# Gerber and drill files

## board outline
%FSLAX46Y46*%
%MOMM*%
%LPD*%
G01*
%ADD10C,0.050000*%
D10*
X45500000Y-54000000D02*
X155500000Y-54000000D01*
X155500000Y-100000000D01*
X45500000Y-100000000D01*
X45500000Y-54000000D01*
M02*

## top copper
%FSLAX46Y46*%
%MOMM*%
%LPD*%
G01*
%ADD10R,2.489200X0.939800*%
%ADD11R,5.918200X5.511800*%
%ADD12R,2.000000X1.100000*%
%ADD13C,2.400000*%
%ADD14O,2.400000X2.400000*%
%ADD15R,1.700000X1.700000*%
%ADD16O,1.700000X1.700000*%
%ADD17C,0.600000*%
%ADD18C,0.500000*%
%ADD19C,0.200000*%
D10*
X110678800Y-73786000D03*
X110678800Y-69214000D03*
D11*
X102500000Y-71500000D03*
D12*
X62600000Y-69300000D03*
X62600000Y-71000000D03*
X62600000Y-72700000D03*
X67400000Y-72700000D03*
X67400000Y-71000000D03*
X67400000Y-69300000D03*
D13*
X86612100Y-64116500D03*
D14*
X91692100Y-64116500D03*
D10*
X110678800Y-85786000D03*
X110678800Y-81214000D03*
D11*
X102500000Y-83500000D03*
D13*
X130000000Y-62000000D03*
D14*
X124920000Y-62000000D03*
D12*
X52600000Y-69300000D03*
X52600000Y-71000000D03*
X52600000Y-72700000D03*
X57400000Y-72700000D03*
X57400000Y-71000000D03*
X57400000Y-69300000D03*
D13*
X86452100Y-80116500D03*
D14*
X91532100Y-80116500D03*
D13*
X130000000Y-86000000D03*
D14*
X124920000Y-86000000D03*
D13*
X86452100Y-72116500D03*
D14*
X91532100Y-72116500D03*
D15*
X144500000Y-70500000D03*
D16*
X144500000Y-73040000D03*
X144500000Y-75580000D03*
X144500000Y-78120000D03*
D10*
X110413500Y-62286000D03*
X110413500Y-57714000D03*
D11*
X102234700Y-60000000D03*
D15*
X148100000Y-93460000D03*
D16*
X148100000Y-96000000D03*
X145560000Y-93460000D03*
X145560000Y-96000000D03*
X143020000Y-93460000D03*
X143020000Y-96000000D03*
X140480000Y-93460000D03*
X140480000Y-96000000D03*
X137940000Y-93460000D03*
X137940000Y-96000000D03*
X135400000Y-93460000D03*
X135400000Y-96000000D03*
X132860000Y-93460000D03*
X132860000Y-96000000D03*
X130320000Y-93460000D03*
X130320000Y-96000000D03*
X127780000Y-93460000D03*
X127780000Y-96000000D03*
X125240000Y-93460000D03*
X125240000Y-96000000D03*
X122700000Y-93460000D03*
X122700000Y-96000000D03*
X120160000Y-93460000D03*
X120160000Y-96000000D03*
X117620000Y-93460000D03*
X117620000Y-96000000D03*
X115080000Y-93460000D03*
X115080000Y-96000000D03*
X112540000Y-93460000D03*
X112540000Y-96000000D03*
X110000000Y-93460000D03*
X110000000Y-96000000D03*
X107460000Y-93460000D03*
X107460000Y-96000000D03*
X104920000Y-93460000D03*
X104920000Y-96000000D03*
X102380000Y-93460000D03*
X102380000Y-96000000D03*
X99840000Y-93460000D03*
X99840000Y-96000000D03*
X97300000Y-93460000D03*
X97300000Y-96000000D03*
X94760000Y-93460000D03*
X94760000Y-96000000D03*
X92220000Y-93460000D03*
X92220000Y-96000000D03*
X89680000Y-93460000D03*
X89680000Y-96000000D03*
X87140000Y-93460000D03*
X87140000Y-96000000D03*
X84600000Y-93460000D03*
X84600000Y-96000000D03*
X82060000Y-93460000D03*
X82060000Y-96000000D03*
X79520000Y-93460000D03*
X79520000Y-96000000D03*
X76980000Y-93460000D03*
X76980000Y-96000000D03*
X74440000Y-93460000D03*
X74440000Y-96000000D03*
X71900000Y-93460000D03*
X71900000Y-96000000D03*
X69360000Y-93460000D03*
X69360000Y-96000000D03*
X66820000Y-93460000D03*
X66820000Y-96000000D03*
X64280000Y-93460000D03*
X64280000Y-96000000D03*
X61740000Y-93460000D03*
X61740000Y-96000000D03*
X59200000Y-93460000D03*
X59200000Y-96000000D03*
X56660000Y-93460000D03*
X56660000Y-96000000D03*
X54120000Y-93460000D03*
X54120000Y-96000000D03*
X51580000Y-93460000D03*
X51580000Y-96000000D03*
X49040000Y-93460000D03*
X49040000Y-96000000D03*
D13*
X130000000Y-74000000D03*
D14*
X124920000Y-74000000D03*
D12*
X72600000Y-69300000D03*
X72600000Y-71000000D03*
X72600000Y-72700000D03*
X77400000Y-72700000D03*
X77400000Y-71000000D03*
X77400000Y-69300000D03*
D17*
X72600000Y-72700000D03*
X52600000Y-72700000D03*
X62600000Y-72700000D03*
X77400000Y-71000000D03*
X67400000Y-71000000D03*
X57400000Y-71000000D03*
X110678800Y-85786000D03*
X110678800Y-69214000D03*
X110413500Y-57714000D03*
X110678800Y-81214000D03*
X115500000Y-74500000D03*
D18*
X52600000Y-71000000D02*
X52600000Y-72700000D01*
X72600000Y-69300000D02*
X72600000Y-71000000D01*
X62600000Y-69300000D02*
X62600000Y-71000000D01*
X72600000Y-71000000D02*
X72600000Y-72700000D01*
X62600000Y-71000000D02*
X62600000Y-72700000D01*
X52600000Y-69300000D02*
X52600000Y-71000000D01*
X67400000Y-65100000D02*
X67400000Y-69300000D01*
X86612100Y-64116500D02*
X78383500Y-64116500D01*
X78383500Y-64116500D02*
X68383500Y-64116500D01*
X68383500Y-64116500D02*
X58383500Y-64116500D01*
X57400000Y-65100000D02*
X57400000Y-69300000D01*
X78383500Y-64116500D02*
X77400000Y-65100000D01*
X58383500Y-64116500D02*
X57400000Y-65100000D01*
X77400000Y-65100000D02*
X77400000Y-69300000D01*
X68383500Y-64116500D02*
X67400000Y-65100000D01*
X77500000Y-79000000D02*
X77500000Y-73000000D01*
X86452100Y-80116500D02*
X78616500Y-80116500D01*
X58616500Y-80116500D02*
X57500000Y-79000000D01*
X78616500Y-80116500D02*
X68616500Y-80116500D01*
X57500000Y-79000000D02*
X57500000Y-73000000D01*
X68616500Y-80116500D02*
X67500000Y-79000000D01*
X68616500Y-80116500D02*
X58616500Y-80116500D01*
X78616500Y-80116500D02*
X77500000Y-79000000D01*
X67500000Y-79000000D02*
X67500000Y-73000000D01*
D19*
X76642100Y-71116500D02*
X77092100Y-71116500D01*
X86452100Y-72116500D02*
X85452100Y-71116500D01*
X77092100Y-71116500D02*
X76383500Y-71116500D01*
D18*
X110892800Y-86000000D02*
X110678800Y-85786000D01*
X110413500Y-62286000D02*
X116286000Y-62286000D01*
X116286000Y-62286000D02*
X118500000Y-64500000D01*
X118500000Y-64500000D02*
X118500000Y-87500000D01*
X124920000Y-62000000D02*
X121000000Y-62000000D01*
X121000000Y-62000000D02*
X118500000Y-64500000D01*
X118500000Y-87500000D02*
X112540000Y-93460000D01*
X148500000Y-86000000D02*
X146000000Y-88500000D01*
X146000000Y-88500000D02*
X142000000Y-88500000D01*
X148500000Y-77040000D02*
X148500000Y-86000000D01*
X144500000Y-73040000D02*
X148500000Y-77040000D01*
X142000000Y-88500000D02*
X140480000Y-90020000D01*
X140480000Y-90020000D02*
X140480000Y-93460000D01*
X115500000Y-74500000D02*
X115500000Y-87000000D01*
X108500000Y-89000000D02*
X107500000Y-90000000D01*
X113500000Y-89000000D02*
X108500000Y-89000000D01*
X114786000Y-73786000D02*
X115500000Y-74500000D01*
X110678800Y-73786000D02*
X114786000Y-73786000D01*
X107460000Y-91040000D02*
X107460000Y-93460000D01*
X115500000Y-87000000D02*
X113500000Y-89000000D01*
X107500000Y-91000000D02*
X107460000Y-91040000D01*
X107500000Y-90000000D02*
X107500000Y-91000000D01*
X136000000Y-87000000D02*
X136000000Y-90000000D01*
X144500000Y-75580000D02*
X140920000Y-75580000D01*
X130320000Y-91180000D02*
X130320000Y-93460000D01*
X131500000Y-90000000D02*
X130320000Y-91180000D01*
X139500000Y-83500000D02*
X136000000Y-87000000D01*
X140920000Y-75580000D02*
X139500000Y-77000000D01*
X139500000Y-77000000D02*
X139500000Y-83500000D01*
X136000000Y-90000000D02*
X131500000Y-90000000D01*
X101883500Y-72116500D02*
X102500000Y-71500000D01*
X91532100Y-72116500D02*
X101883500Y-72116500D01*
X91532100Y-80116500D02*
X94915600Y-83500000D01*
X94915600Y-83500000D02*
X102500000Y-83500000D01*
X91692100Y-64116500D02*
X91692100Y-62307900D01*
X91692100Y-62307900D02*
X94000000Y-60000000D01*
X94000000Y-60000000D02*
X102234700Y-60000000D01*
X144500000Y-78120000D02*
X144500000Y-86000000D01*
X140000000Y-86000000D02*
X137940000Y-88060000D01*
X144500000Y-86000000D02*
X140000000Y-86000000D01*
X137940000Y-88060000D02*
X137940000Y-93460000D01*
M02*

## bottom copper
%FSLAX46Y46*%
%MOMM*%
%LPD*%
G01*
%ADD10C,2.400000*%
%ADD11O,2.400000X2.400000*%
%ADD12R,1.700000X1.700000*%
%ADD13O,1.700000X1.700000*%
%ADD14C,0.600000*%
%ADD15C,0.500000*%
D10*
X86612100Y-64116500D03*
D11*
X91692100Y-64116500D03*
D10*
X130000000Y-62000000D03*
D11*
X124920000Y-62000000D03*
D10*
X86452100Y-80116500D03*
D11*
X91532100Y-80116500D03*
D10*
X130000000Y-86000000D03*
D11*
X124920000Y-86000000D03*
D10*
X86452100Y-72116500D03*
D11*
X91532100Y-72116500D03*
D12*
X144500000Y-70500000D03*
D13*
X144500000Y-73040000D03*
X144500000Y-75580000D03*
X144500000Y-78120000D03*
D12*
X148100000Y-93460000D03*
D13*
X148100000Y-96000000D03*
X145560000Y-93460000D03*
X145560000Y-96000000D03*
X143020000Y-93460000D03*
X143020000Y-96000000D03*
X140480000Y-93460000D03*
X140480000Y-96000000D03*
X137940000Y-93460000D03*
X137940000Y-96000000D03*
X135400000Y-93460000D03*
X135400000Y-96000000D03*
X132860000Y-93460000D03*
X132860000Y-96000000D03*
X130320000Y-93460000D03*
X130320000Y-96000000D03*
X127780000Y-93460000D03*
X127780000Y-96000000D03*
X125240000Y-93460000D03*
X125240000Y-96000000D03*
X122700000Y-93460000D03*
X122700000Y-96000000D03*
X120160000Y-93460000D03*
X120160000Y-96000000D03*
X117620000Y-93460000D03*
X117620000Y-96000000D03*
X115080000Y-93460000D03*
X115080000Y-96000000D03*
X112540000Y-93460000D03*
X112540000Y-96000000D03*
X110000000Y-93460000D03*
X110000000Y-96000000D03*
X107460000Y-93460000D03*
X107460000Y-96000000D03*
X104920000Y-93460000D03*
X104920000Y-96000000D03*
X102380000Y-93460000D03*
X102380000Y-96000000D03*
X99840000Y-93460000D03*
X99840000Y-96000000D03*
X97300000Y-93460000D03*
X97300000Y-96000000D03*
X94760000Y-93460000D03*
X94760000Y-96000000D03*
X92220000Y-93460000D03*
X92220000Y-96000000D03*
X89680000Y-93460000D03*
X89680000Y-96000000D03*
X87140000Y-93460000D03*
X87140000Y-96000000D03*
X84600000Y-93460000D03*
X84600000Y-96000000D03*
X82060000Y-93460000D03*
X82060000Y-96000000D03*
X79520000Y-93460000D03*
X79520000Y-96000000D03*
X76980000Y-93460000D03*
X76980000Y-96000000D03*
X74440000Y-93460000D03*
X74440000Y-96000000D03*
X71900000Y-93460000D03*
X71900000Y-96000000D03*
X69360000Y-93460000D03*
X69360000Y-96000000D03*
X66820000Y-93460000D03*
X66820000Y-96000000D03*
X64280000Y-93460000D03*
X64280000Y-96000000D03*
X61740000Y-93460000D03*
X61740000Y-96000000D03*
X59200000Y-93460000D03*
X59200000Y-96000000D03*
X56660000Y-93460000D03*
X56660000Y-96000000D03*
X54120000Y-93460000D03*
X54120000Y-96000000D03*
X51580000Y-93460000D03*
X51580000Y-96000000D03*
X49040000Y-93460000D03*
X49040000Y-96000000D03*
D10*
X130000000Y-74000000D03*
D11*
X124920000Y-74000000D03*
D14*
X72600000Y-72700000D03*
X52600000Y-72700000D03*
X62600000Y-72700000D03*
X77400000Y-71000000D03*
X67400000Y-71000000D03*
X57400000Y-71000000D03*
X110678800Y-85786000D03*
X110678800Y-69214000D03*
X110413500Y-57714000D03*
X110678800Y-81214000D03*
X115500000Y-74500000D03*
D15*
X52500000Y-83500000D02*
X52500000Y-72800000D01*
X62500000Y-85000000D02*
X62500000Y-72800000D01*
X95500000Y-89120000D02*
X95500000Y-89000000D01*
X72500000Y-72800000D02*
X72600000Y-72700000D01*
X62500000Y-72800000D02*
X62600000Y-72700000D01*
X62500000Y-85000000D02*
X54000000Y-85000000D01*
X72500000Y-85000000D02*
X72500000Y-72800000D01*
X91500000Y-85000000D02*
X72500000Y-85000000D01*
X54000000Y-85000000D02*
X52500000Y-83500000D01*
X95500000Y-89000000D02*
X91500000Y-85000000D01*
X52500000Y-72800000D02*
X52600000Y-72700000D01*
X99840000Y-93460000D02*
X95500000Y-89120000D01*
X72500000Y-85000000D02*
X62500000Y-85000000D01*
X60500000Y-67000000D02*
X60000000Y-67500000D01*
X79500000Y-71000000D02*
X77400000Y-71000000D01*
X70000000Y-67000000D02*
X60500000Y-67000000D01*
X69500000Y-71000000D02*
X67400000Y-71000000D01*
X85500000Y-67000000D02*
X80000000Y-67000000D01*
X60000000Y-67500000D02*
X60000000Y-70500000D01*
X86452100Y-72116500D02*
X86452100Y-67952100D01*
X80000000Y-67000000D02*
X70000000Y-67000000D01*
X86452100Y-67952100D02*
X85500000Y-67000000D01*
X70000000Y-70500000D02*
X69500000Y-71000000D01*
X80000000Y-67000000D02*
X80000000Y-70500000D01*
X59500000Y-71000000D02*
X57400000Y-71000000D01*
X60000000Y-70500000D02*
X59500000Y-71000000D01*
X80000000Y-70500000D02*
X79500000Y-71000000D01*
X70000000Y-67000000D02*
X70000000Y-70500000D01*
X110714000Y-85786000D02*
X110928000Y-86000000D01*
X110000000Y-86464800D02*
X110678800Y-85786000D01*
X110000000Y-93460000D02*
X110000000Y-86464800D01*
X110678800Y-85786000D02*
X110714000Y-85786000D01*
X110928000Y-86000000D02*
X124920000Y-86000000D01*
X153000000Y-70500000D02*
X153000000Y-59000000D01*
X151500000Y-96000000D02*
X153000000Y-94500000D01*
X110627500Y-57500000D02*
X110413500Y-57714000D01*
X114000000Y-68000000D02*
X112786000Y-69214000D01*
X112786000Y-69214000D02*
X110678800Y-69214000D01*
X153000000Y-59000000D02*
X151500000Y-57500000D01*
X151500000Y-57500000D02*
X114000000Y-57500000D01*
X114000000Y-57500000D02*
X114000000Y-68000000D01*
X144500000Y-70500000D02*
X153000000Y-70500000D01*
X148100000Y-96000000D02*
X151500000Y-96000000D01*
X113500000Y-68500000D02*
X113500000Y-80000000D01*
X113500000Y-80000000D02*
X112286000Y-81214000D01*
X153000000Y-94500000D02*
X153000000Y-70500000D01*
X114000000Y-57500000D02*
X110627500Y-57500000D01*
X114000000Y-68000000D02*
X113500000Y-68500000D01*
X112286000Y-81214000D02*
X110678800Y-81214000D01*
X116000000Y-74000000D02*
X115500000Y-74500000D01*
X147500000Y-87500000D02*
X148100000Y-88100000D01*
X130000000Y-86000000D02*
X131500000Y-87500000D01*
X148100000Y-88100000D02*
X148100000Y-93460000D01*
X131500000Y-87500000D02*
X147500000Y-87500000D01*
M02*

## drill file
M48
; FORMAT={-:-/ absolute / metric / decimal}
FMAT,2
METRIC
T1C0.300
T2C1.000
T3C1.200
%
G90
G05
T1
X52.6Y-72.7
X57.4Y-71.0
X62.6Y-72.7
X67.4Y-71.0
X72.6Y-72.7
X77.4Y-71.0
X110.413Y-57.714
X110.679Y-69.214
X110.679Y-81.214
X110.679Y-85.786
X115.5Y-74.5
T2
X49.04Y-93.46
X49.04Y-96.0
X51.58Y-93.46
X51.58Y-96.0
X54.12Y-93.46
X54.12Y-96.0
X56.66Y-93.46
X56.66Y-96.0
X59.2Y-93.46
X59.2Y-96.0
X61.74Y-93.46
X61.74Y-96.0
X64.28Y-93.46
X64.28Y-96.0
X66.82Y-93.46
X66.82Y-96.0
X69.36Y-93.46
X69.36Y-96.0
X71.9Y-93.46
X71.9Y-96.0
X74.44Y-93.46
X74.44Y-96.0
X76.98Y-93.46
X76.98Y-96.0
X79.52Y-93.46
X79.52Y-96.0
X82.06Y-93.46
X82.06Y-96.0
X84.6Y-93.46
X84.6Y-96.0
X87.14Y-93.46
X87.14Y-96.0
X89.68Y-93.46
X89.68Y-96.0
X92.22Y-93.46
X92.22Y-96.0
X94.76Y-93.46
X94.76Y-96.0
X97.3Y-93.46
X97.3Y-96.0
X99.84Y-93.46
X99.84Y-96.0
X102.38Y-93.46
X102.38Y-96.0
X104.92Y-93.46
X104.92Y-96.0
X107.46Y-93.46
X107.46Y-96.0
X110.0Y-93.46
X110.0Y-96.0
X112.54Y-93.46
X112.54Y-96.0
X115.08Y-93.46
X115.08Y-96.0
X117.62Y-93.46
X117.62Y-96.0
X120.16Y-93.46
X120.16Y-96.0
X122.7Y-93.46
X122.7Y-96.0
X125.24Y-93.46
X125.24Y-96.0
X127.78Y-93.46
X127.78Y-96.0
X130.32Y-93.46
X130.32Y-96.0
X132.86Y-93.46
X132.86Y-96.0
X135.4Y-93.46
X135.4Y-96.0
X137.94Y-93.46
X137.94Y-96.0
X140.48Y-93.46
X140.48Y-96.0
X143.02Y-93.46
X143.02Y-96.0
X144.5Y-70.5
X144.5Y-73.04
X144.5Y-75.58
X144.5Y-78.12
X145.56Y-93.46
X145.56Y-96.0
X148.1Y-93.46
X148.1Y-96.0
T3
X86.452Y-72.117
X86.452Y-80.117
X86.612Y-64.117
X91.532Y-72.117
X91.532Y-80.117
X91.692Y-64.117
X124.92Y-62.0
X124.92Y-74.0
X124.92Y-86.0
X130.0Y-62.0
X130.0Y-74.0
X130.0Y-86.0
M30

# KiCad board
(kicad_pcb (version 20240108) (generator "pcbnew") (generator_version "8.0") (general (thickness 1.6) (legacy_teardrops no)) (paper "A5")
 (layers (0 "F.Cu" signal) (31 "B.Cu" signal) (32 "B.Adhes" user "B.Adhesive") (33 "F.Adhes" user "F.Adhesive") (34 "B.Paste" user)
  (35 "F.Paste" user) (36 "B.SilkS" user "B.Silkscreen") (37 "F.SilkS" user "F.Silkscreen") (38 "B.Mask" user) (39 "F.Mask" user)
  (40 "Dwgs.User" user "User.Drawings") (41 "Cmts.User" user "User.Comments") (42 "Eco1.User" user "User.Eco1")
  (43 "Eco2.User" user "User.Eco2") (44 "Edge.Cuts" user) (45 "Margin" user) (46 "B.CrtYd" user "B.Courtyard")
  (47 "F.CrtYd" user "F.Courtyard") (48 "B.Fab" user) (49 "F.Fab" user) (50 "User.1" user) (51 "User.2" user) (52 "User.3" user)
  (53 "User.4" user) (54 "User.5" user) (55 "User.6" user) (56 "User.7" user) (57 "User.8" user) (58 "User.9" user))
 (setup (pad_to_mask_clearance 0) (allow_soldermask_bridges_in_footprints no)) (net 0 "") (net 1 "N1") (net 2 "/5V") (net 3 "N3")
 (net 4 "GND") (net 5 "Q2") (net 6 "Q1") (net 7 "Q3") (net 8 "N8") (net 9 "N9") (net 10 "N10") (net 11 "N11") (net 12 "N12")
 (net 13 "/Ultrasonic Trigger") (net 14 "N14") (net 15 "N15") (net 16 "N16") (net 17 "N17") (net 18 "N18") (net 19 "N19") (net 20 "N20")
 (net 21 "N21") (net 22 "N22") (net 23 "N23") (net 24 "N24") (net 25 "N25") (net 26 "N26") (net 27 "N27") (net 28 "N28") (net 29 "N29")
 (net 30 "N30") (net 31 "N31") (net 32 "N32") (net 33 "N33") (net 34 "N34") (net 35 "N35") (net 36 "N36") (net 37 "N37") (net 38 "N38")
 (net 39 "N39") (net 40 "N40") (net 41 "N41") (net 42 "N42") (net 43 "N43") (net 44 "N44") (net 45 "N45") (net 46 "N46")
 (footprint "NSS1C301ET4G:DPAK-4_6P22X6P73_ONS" (layer "F.Cu") (at 104.2653 71.5 90)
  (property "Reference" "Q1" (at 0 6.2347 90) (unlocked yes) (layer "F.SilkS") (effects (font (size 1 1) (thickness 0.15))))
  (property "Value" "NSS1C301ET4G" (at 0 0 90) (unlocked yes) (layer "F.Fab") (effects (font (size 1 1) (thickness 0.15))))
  (pad "1" smd rect (at -2.286 6.4135 90) (size 0.9398 2.4892) (layers "F.Cu" "F.Paste" "F.Mask") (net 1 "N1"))
  (pad "2" smd rect (at 2.286 6.4135 90) (size 0.9398 2.4892) (layers "F.Cu" "F.Paste" "F.Mask") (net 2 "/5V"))
  (pad "3" smd rect (at 0 -1.7653 90) (size 5.5118 5.9182) (layers "F.Cu" "F.Paste" "F.Mask") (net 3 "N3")))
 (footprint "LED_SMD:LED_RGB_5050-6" (layer "F.Cu") (at 65 71)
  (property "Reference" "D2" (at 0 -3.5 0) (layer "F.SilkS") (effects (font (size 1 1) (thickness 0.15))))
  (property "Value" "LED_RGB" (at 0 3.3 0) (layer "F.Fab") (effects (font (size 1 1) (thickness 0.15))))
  (pad "1" smd rect (at -2.4 -1.7 90) (size 1.1 2) (layers "F.Cu" "F.Paste" "F.Mask") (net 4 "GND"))
  (pad "2" smd rect (at -2.4 0 90) (size 1.1 2) (layers "F.Cu" "F.Paste" "F.Mask") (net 4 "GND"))
  (pad "3" smd rect (at -2.4 1.7 90) (size 1.1 2) (layers "F.Cu" "F.Paste" "F.Mask") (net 4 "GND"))
  (pad "4" smd rect (at 2.4 1.7 90) (size 1.1 2) (layers "F.Cu" "F.Paste" "F.Mask") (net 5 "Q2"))
  (pad "5" smd rect (at 2.4 0 90) (size 1.1 2) (layers "F.Cu" "F.Paste" "F.Mask") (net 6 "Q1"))
  (pad "6" smd rect (at 2.4 -1.7 90) (size 1.1 2) (layers "F.Cu" "F.Paste" "F.Mask") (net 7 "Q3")))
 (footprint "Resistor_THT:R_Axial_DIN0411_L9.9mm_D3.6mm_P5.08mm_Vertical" (layer "F.Cu") (at 86.6121 64.1165)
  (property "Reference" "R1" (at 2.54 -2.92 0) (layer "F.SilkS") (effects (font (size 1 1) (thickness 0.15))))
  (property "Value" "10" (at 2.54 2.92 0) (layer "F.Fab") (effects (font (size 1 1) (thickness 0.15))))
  (pad "1" thru_hole circle (at 0 0) (size 2.4 2.4) (drill 1.2) (layers "*.Cu" "*.Mask") (remove_unused_layers no) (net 7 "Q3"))
  (pad "2" thru_hole oval (at 5.08 0) (size 2.4 2.4) (drill 1.2) (layers "*.Cu" "*.Mask") (remove_unused_layers no) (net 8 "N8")))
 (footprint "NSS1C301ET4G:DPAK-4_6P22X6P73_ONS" (layer "F.Cu") (at 104.2653 83.5 90)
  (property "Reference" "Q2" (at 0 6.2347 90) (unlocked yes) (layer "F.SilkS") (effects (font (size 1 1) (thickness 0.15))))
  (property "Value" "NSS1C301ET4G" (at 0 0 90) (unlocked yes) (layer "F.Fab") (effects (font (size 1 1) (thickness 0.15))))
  (pad "1" smd rect (at -2.286 6.4135 90) (size 0.9398 2.4892) (layers "F.Cu" "F.Paste" "F.Mask") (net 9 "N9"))
  (pad "2" smd rect (at 2.286 6.4135 90) (size 0.9398 2.4892) (layers "F.Cu" "F.Paste" "F.Mask") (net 2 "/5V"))
  (pad "3" smd rect (at 0 -1.7653 90) (size 5.5118 5.9182) (layers "F.Cu" "F.Paste" "F.Mask") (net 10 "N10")))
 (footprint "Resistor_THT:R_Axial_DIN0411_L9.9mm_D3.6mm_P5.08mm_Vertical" (layer "F.Cu") (at 130 62 180)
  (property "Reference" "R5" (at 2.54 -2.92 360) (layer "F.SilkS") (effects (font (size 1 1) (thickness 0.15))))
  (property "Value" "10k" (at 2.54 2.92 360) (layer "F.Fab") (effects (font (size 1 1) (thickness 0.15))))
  (pad "1" thru_hole circle (at 0 0 180) (size 2.4 2.4) (drill 1.2) (layers "*.Cu" "*.Mask") (remove_unused_layers no) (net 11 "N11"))
  (pad "2" thru_hole oval (at 5.08 0 180) (size 2.4 2.4) (drill 1.2) (layers "*.Cu" "*.Mask") (remove_unused_layers no) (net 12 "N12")))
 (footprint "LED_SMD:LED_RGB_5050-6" (layer "F.Cu") (at 55 71)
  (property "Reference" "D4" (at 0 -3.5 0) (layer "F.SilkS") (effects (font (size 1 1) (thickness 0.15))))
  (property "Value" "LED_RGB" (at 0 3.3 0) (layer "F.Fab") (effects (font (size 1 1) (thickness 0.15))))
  (pad "1" smd rect (at -2.4 -1.7 90) (size 1.1 2) (layers "F.Cu" "F.Paste" "F.Mask") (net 4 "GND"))
  (pad "2" smd rect (at -2.4 0 90) (size 1.1 2) (layers "F.Cu" "F.Paste" "F.Mask") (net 4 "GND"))
  (pad "3" smd rect (at -2.4 1.7 90) (size 1.1 2) (layers "F.Cu" "F.Paste" "F.Mask") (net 4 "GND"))
  (pad "4" smd rect (at 2.4 1.7 90) (size 1.1 2) (layers "F.Cu" "F.Paste" "F.Mask") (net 5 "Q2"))
  (pad "5" smd rect (at 2.4 0 90) (size 1.1 2) (layers "F.Cu" "F.Paste" "F.Mask") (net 6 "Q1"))
  (pad "6" smd rect (at 2.4 -1.7 90) (size 1.1 2) (layers "F.Cu" "F.Paste" "F.Mask") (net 7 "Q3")))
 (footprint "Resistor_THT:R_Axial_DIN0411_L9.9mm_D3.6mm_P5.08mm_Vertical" (layer "F.Cu") (at 86.4521 80.1165)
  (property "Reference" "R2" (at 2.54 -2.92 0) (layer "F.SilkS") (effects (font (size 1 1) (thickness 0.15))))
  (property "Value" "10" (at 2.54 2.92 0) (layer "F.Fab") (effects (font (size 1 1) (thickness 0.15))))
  (pad "1" thru_hole circle (at 0 0) (size 2.4 2.4) (drill 1.2) (layers "*.Cu" "*.Mask") (remove_unused_layers no) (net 5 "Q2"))
  (pad "2" thru_hole oval (at 5.08 0) (size 2.4 2.4) (drill 1.2) (layers "*.Cu" "*.Mask") (remove_unused_layers no) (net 10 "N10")))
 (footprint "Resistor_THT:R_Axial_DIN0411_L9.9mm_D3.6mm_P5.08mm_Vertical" (layer "F.Cu") (at 130 86 180)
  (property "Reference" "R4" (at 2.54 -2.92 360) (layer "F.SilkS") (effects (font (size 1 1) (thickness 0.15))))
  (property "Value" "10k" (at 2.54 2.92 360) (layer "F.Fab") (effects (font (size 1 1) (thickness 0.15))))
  (pad "1" thru_hole circle (at 0 0 180) (size 2.4 2.4) (drill 1.2) (layers "*.Cu" "*.Mask") (remove_unused_layers no) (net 11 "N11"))
  (pad "2" thru_hole oval (at 5.08 0 180) (size 2.4 2.4) (drill 1.2) (layers "*.Cu" "*.Mask") (remove_unused_layers no) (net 9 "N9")))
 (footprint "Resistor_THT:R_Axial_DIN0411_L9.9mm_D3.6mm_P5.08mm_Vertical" (layer "F.Cu") (at 86.4521 72.1165)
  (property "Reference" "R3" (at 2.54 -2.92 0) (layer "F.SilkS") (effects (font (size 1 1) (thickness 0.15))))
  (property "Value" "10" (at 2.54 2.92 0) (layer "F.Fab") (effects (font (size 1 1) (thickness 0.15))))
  (pad "1" thru_hole circle (at 0 0) (size 2.4 2.4) (drill 1.2) (layers "*.Cu" "*.Mask") (remove_unused_layers no) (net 6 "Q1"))
  (pad "2" thru_hole oval (at 5.08 0) (size 2.4 2.4) (drill 1.2) (layers "*.Cu" "*.Mask") (remove_unused_layers no) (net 3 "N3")))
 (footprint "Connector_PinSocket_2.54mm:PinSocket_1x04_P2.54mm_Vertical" (layer "F.Cu") (at 144.5 70.5)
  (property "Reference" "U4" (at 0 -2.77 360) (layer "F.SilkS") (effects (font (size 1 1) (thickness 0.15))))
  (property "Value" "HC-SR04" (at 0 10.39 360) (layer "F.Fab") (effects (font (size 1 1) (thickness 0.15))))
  (pad "1" thru_hole rect (at 0 0) (size 1.7 1.7) (drill 1) (layers "*.Cu" "*.Mask") (remove_unused_layers no) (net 2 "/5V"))
  (pad "2" thru_hole oval (at 0 2.54) (size 1.7 1.7) (drill 1) (layers "*.Cu" "*.Mask") (remove_unused_layers no)
   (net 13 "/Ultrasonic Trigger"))
  (pad "3" thru_hole oval (at 0 5.08) (size 1.7 1.7) (drill 1) (layers "*.Cu" "*.Mask") (remove_unused_layers no) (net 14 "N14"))
  (pad "4" thru_hole oval (at 0 7.62) (size 1.7 1.7) (drill 1) (layers "*.Cu" "*.Mask") (remove_unused_layers no) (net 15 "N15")))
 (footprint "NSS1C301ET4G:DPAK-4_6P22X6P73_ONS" (layer "F.Cu") (at 104 60 90)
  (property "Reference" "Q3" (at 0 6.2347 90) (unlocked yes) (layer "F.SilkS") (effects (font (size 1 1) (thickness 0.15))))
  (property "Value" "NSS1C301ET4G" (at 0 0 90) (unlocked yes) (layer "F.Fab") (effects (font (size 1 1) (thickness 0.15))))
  (pad "1" smd rect (at -2.286 6.4135 90) (size 0.9398 2.4892) (layers "F.Cu" "F.Paste" "F.Mask") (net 12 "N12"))
  (pad "2" smd rect (at 2.286 6.4135 90) (size 0.9398 2.4892) (layers "F.Cu" "F.Paste" "F.Mask") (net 2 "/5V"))
  (pad "3" smd rect (at 0 -1.7653 90) (size 5.5118 5.9182) (layers "F.Cu" "F.Paste" "F.Mask") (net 8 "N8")))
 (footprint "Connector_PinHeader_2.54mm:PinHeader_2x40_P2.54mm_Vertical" (layer "F.Cu") (at 148.1 93.46 -90)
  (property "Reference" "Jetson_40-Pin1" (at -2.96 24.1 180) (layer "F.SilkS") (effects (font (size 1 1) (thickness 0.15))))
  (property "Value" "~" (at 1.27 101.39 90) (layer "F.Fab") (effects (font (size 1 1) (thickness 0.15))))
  (pad "1" thru_hole rect (at 0 0 270) (size 1.7 1.7) (drill 1) (layers "*.Cu" "*.Mask") (remove_unused_layers no) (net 11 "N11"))
  (pad "2" thru_hole oval (at 2.54 0 270) (size 1.7 1.7) (drill 1) (layers "*.Cu" "*.Mask") (remove_unused_layers no) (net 2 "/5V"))
  (pad "3" thru_hole oval (at 0 2.54 270) (size 1.7 1.7) (drill 1) (layers "*.Cu" "*.Mask") (remove_unused_layers no) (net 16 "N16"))
  (pad "4" thru_hole oval (at 2.54 2.54 270) (size 1.7 1.7) (drill 1) (layers "*.Cu" "*.Mask") (remove_unused_layers no) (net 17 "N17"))
  (pad "5" thru_hole oval (at 0 5.08 270) (size 1.7 1.7) (drill 1) (layers "*.Cu" "*.Mask") (remove_unused_layers no) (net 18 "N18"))
  (pad "6" thru_hole oval (at 2.54 5.08 270) (size 1.7 1.7) (drill 1) (layers "*.Cu" "*.Mask") (remove_unused_layers no) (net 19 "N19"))
  (pad "7" thru_hole oval (at 0 7.62 270) (size 1.7 1.7) (drill 1) (layers "*.Cu" "*.Mask") (remove_unused_layers no)
   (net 13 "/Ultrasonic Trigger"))
  (pad "8" thru_hole oval (at 2.54 7.62 270) (size 1.7 1.7) (drill 1) (layers "*.Cu" "*.Mask") (remove_unused_layers no) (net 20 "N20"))
  (pad "9" thru_hole oval (at 0 10.16 270) (size 1.7 1.7) (drill 1) (layers "*.Cu" "*.Mask") (remove_unused_layers no) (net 15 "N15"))
  (pad "10" thru_hole oval (at 2.54 10.16 270) (size 1.7 1.7) (drill 1) (layers "*.Cu" "*.Mask") (remove_unused_layers no) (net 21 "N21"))
  (pad "11" thru_hole oval (at 0 12.7 270) (size 1.7 1.7) (drill 1) (layers "*.Cu" "*.Mask") (remove_unused_layers no) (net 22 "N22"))
  (pad "12" thru_hole oval (at 2.54 12.7 270) (size 1.7 1.7) (drill 1) (layers "*.Cu" "*.Mask") (remove_unused_layers no) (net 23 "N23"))
  (pad "13" thru_hole oval (at 0 15.24 270) (size 1.7 1.7) (drill 1) (layers "*.Cu" "*.Mask") (remove_unused_layers no) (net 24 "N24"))
  (pad "14" thru_hole oval (at 2.54 15.24 270) (size 1.7 1.7) (drill 1) (layers "*.Cu" "*.Mask") (remove_unused_layers no) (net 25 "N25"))
  (pad "15" thru_hole oval (at 0 17.78 270) (size 1.7 1.7) (drill 1) (layers "*.Cu" "*.Mask") (remove_unused_layers no) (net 14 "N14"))
  (pad "16" thru_hole oval (at 2.54 17.78 270) (size 1.7 1.7) (drill 1) (layers "*.Cu" "*.Mask") (remove_unused_layers no) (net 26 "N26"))
  (pad "17" thru_hole oval (at 0 20.32 270) (size 1.7 1.7) (drill 1) (layers "*.Cu" "*.Mask") (remove_unused_layers no) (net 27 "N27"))
  (pad "18" thru_hole oval (at 2.54 20.32 270) (size 1.7 1.7) (drill 1) (layers "*.Cu" "*.Mask") (remove_unused_layers no) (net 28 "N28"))
  (pad "19" thru_hole oval (at 0 22.86 270) (size 1.7 1.7) (drill 1) (layers "*.Cu" "*.Mask") (remove_unused_layers no) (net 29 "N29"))
  (pad "20" thru_hole oval (at 2.54 22.86 270) (size 1.7 1.7) (drill 1) (layers "*.Cu" "*.Mask") (remove_unused_layers no) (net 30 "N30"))
  (pad "21" thru_hole oval (at 0 25.4 270) (size 1.7 1.7) (drill 1) (layers "*.Cu" "*.Mask") (remove_unused_layers no) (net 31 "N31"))
  (pad "22" thru_hole oval (at 2.54 25.4 270) (size 1.7 1.7) (drill 1) (layers "*.Cu" "*.Mask") (remove_unused_layers no) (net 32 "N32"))
  (pad "23" thru_hole oval (at 0 27.94 270) (size 1.7 1.7) (drill 1) (layers "*.Cu" "*.Mask") (remove_unused_layers no) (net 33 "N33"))
  (pad "24" thru_hole oval (at 2.54 27.94 270) (size 1.7 1.7) (drill 1) (layers "*.Cu" "*.Mask") (remove_unused_layers no) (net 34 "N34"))
  (pad "25" thru_hole oval (at 0 30.48 270) (size 1.7 1.7) (drill 1) (layers "*.Cu" "*.Mask") (remove_unused_layers no) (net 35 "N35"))
  (pad "26" thru_hole oval (at 2.54 30.48 270) (size 1.7 1.7) (drill 1) (layers "*.Cu" "*.Mask") (remove_unused_layers no) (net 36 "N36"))
  (pad "27" thru_hole oval (at 0 33.02 270) (size 1.7 1.7) (drill 1) (layers "*.Cu" "*.Mask") (remove_unused_layers no) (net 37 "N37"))
  (pad "28" thru_hole oval (at 2.54 33.02 270) (size 1.7 1.7) (drill 1) (layers "*.Cu" "*.Mask") (remove_unused_layers no) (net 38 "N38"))
  (pad "29" thru_hole oval (at 0 35.56 270) (size 1.7 1.7) (drill 1) (layers "*.Cu" "*.Mask") (remove_unused_layers no) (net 12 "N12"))
  (pad "30" thru_hole oval (at 2.54 35.56 270) (size 1.7 1.7) (drill 1) (layers "*.Cu" "*.Mask") (remove_unused_layers no) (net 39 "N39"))
  (pad "31" thru_hole oval (at 0 38.1 270) (size 1.7 1.7) (drill 1) (layers "*.Cu" "*.Mask") (remove_unused_layers no) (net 9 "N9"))
  (pad "32" thru_hole oval (at 2.54 38.1 270) (size 1.7 1.7) (drill 1) (layers "*.Cu" "*.Mask") (remove_unused_layers no) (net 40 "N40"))
  (pad "33" thru_hole oval (at 0 40.64 270) (size 1.7 1.7) (drill 1) (layers "*.Cu" "*.Mask") (remove_unused_layers no) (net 1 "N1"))
  (pad "34" thru_hole oval (at 2.54 40.64 270) (size 1.7 1.7) (drill 1) (layers "*.Cu" "*.Mask") (remove_unused_layers no) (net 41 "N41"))
  (pad "35" thru_hole oval (at 0 43.18 270) (size 1.7 1.7) (drill 1) (layers "*.Cu" "*.Mask") (remove_unused_layers no) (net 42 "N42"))
  (pad "36" thru_hole oval (at 2.54 43.18 270) (size 1.7 1.7) (drill 1) (layers "*.Cu" "*.Mask") (remove_unused_layers no) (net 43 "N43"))
  (pad "37" thru_hole oval (at 0 45.72 270) (size 1.7 1.7) (drill 1) (layers "*.Cu" "*.Mask") (remove_unused_layers no) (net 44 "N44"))
  (pad "38" thru_hole oval (at 2.54 45.72 270) (size 1.7 1.7) (drill 1) (layers "*.Cu" "*.Mask") (remove_unused_layers no) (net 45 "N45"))
  (pad "39" thru_hole oval (at 0 48.26 270) (size 1.7 1.7) (drill 1) (layers "*.Cu" "*.Mask") (remove_unused_layers no) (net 4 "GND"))
  (pad "40" thru_hole oval (at 2.54 48.26 270) (size 1.7 1.7) (drill 1) (layers "*.Cu" "*.Mask") (remove_unused_layers no) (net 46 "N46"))
  (pad "41" thru_hole oval (at 0 50.8 270) (size 1.7 1.7) (drill 1) (layers "*.Cu" "*.Mask") (remove_unused_layers no))
  (pad "42" thru_hole oval (at 2.54 50.8 270) (size 1.7 1.7) (drill 1) (layers "*.Cu" "*.Mask") (remove_unused_layers no))
  (pad "43" thru_hole oval (at 0 53.34 270) (size 1.7 1.7) (drill 1) (layers "*.Cu" "*.Mask") (remove_unused_layers no))
  (pad "44" thru_hole oval (at 2.54 53.34 270) (size 1.7 1.7) (drill 1) (layers "*.Cu" "*.Mask") (remove_unused_layers no))
  (pad "45" thru_hole oval (at 0 55.88 270) (size 1.7 1.7) (drill 1) (layers "*.Cu" "*.Mask") (remove_unused_layers no))
  (pad "46" thru_hole oval (at 2.54 55.88 270) (size 1.7 1.7) (drill 1) (layers "*.Cu" "*.Mask") (remove_unused_layers no))
  (pad "47" thru_hole oval (at 0 58.42 270) (size 1.7 1.7) (drill 1) (layers "*.Cu" "*.Mask") (remove_unused_layers no))
  (pad "48" thru_hole oval (at 2.54 58.42 270) (size 1.7 1.7) (drill 1) (layers "*.Cu" "*.Mask") (remove_unused_layers no))
  (pad "49" thru_hole oval (at 0 60.96 270) (size 1.7 1.7) (drill 1) (layers "*.Cu" "*.Mask") (remove_unused_layers no))
  (pad "50" thru_hole oval (at 2.54 60.96 270) (size 1.7 1.7) (drill 1) (layers "*.Cu" "*.Mask") (remove_unused_layers no))
  (pad "51" thru_hole oval (at 0 63.5 270) (size 1.7 1.7) (drill 1) (layers "*.Cu" "*.Mask") (remove_unused_layers no))
  (pad "52" thru_hole oval (at 2.54 63.5 270) (size 1.7 1.7) (drill 1) (layers "*.Cu" "*.Mask") (remove_unused_layers no))
  (pad "53" thru_hole oval (at 0 66.04 270) (size 1.7 1.7) (drill 1) (layers "*.Cu" "*.Mask") (remove_unused_layers no))
  (pad "54" thru_hole oval (at 2.54 66.04 270) (size 1.7 1.7) (drill 1) (layers "*.Cu" "*.Mask") (remove_unused_layers no))
  (pad "55" thru_hole oval (at 0 68.58 270) (size 1.7 1.7) (drill 1) (layers "*.Cu" "*.Mask") (remove_unused_layers no))
  (pad "56" thru_hole oval (at 2.54 68.58 270) (size 1.7 1.7) (drill 1) (layers "*.Cu" "*.Mask") (remove_unused_layers no))
  (pad "57" thru_hole oval (at 0 71.12 270) (size 1.7 1.7) (drill 1) (layers "*.Cu" "*.Mask") (remove_unused_layers no))
  (pad "58" thru_hole oval (at 2.54 71.12 270) (size 1.7 1.7) (drill 1) (layers "*.Cu" "*.Mask") (remove_unused_layers no))
  (pad "59" thru_hole oval (at 0 73.66 270) (size 1.7 1.7) (drill 1) (layers "*.Cu" "*.Mask") (remove_unused_layers no))
  (pad "60" thru_hole oval (at 2.54 73.66 270) (size 1.7 1.7) (drill 1) (layers "*.Cu" "*.Mask") (remove_unused_layers no))
  (pad "61" thru_hole oval (at 0 76.2 270) (size 1.7 1.7) (drill 1) (layers "*.Cu" "*.Mask") (remove_unused_layers no))
  (pad "62" thru_hole oval (at 2.54 76.2 270) (size 1.7 1.7) (drill 1) (layers "*.Cu" "*.Mask") (remove_unused_layers no))
  (pad "63" thru_hole oval (at 0 78.74 270) (size 1.7 1.7) (drill 1) (layers "*.Cu" "*.Mask") (remove_unused_layers no))
  (pad "64" thru_hole oval (at 2.54 78.74 270) (size 1.7 1.7) (drill 1) (layers "*.Cu" "*.Mask") (remove_unused_layers no))
  (pad "65" thru_hole oval (at 0 81.28 270) (size 1.7 1.7) (drill 1) (layers "*.Cu" "*.Mask") (remove_unused_layers no))
  (pad "66" thru_hole oval (at 2.54 81.28 270) (size 1.7 1.7) (drill 1) (layers "*.Cu" "*.Mask") (remove_unused_layers no))
  (pad "67" thru_hole oval (at 0 83.82 270) (size 1.7 1.7) (drill 1) (layers "*.Cu" "*.Mask") (remove_unused_layers no))
  (pad "68" thru_hole oval (at 2.54 83.82 270) (size 1.7 1.7) (drill 1) (layers "*.Cu" "*.Mask") (remove_unused_layers no))
  (pad "69" thru_hole oval (at 0 86.36 270) (size 1.7 1.7) (drill 1) (layers "*.Cu" "*.Mask") (remove_unused_layers no))
  (pad "70" thru_hole oval (at 2.54 86.36 270) (size 1.7 1.7) (drill 1) (layers "*.Cu" "*.Mask") (remove_unused_layers no))
  (pad "71" thru_hole oval (at 0 88.9 270) (size 1.7 1.7) (drill 1) (layers "*.Cu" "*.Mask") (remove_unused_layers no))
  (pad "72" thru_hole oval (at 2.54 88.9 270) (size 1.7 1.7) (drill 1) (layers "*.Cu" "*.Mask") (remove_unused_layers no))
  (pad "73" thru_hole oval (at 0 91.44 270) (size 1.7 1.7) (drill 1) (layers "*.Cu" "*.Mask") (remove_unused_layers no))
  (pad "74" thru_hole oval (at 2.54 91.44 270) (size 1.7 1.7) (drill 1) (layers "*.Cu" "*.Mask") (remove_unused_layers no))
  (pad "75" thru_hole oval (at 0 93.98 270) (size 1.7 1.7) (drill 1) (layers "*.Cu" "*.Mask") (remove_unused_layers no))
  (pad "76" thru_hole oval (at 2.54 93.98 270) (size 1.7 1.7) (drill 1) (layers "*.Cu" "*.Mask") (remove_unused_layers no))
  (pad "77" thru_hole oval (at 0 96.52 270) (size 1.7 1.7) (drill 1) (layers "*.Cu" "*.Mask") (remove_unused_layers no))
  (pad "78" thru_hole oval (at 2.54 96.52 270) (size 1.7 1.7) (drill 1) (layers "*.Cu" "*.Mask") (remove_unused_layers no))
  (pad "79" thru_hole oval (at 0 99.06 270) (size 1.7 1.7) (drill 1) (layers "*.Cu" "*.Mask") (remove_unused_layers no))
  (pad "80" thru_hole oval (at 2.54 99.06 270) (size 1.7 1.7) (drill 1) (layers "*.Cu" "*.Mask") (remove_unused_layers no)))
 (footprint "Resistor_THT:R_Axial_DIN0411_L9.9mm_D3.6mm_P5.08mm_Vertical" (layer "F.Cu") (at 130 74 180)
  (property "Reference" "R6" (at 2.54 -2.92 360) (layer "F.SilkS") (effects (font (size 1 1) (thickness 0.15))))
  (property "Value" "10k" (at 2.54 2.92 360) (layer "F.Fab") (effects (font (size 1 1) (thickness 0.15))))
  (pad "1" thru_hole circle (at 0 0 180) (size 2.4 2.4) (drill 1.2) (layers "*.Cu" "*.Mask") (remove_unused_layers no) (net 11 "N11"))
  (pad "2" thru_hole oval (at 5.08 0 180) (size 2.4 2.4) (drill 1.2) (layers "*.Cu" "*.Mask") (remove_unused_layers no) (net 1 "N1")))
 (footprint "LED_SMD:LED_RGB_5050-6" (layer "F.Cu") (at 75 71)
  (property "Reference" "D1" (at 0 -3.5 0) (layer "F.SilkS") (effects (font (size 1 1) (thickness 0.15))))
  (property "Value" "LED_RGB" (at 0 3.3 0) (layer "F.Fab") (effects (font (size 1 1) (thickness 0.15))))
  (pad "1" smd rect (at -2.4 -1.7 90) (size 1.1 2) (layers "F.Cu" "F.Paste" "F.Mask") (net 4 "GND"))
  (pad "2" smd rect (at -2.4 0 90) (size 1.1 2) (layers "F.Cu" "F.Paste" "F.Mask") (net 4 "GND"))
  (pad "3" smd rect (at -2.4 1.7 90) (size 1.1 2) (layers "F.Cu" "F.Paste" "F.Mask") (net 4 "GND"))
  (pad "4" smd rect (at 2.4 1.7 90) (size 1.1 2) (layers "F.Cu" "F.Paste" "F.Mask") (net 5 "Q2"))
  (pad "5" smd rect (at 2.4 0 90) (size 1.1 2) (layers "F.Cu" "F.Paste" "F.Mask") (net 6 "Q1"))
  (pad "6" smd rect (at 2.4 -1.7 90) (size 1.1 2) (layers "F.Cu" "F.Paste" "F.Mask") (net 7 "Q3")))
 (gr_rect (start 45.5 54) (end 155.5 100) (stroke (width 0.05) (type default)) (fill none) (layer "Edge.Cuts"))
 (segment (start 52.6 71) (end 52.6 72.7) (width 0.5) (layer "F.Cu") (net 4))
 (segment (start 72.6 69.3) (end 72.6 71) (width 0.5) (layer "F.Cu") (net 4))
 (segment (start 62.6 69.3) (end 62.6 71) (width 0.5) (layer "F.Cu") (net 4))
 (segment (start 72.6 71) (end 72.6 72.7) (width 0.5) (layer "F.Cu") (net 4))
 (segment (start 62.6 71) (end 62.6 72.7) (width 0.5) (layer "F.Cu") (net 4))
 (segment (start 52.6 69.3) (end 52.6 71) (width 0.5) (layer "F.Cu") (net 4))
 (via (at 72.6 72.7) (size 0.6) (drill 0.3) (layers "F.Cu" "B.Cu") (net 4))
 (via (at 52.6 72.7) (size 0.6) (drill 0.3) (layers "F.Cu" "B.Cu") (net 4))
 (via (at 62.6 72.7) (size 0.6) (drill 0.3) (layers "F.Cu" "B.Cu") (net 4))
 (segment (start 52.5 83.5) (end 52.5 72.8) (width 0.5) (layer "B.Cu") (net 4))
 (segment (start 62.5 85) (end 62.5 72.8) (width 0.5) (layer "B.Cu") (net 4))
 (segment (start 95.5 89.12) (end 95.5 89) (width 0.5) (layer "B.Cu") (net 4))
 (segment (start 72.5 72.8) (end 72.6 72.7) (width 0.5) (layer "B.Cu") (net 4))
 (segment (start 62.5 72.8) (end 62.6 72.7) (width 0.5) (layer "B.Cu") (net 4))
 (segment (start 62.5 85) (end 54 85) (width 0.5) (layer "B.Cu") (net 4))
 (segment (start 72.5 85) (end 72.5 72.8) (width 0.5) (layer "B.Cu") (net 4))
 (segment (start 91.5 85) (end 72.5 85) (width 0.5) (layer "B.Cu") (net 4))
 (segment (start 54 85) (end 52.5 83.5) (width 0.5) (layer "B.Cu") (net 4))
 (segment (start 95.5 89) (end 91.5 85) (width 0.5) (layer "B.Cu") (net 4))
 (segment (start 52.5 72.8) (end 52.6 72.7) (width 0.5) (layer "B.Cu") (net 4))
 (segment (start 99.84 93.46) (end 95.5 89.12) (width 0.5) (layer "B.Cu") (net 4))
 (segment (start 72.5 85) (end 62.5 85) (width 0.5) (layer "B.Cu") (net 4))
 (segment (start 67.4 65.1) (end 67.4 69.3) (width 0.5) (layer "F.Cu") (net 7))
 (segment (start 86.6121 64.1165) (end 78.3835 64.1165) (width 0.5) (layer "F.Cu") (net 7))
 (segment (start 78.3835 64.1165) (end 68.3835 64.1165) (width 0.5) (layer "F.Cu") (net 7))
 (segment (start 68.3835 64.1165) (end 58.3835 64.1165) (width 0.5) (layer "F.Cu") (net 7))
 (segment (start 57.4 65.1) (end 57.4 69.3) (width 0.5) (layer "F.Cu") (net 7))
 (segment (start 78.3835 64.1165) (end 77.4 65.1) (width 0.5) (layer "F.Cu") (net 7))
 (segment (start 58.3835 64.1165) (end 57.4 65.1) (width 0.5) (layer "F.Cu") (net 7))
 (segment (start 77.4 65.1) (end 77.4 69.3) (width 0.5) (layer "F.Cu") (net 7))
 (segment (start 68.3835 64.1165) (end 67.4 65.1) (width 0.5) (layer "F.Cu") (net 7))
 (segment (start 77.5 79) (end 77.5 73) (width 0.5) (layer "F.Cu") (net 5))
 (segment (start 86.4521 80.1165) (end 78.6165 80.1165) (width 0.5) (layer "F.Cu") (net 5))
 (segment (start 58.6165 80.1165) (end 57.5 79) (width 0.5) (layer "F.Cu") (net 5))
 (segment (start 78.6165 80.1165) (end 68.6165 80.1165) (width 0.5) (layer "F.Cu") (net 5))
 (segment (start 57.5 79) (end 57.5 73) (width 0.5) (layer "F.Cu") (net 5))
 (segment (start 68.6165 80.1165) (end 67.5 79) (width 0.5) (layer "F.Cu") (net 5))
 (segment (start 68.6165 80.1165) (end 58.6165 80.1165) (width 0.5) (layer "F.Cu") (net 5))
 (segment (start 78.6165 80.1165) (end 77.5 79) (width 0.5) (layer "F.Cu") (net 5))
 (segment (start 67.5 79) (end 67.5 73) (width 0.5) (layer "F.Cu") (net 5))
 (segment (start 76.6421 71.1165) (end 77.0921 71.1165) (width 0.2) (layer "F.Cu") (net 6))
 (segment (start 86.4521 72.1165) (end 85.4521 71.1165) (width 0.2) (layer "F.Cu") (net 6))
 (segment (start 77.0921 71.1165) (end 76.3835 71.1165) (width 0.2) (layer "F.Cu") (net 6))
 (via (at 77.4 71) (size 0.6) (drill 0.3) (layers "F.Cu" "B.Cu") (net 6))
 (via (at 67.4 71) (size 0.6) (drill 0.3) (layers "F.Cu" "B.Cu") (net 6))
 (via (at 57.4 71) (size 0.6) (drill 0.3) (layers "F.Cu" "B.Cu") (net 6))
 (segment (start 60.5 67) (end 60 67.5) (width 0.5) (layer "B.Cu") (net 6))
 (segment (start 79.5 71) (end 77.4 71) (width 0.5) (layer "B.Cu") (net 6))
 (segment (start 70 67) (end 60.5 67) (width 0.5) (layer "B.Cu") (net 6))
 (segment (start 69.5 71) (end 67.4 71) (width 0.5) (layer "B.Cu") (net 6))
 (segment (start 85.5 67) (end 80 67) (width 0.5) (layer "B.Cu") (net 6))
 (segment (start 60 67.5) (end 60 70.5) (width 0.5) (layer "B.Cu") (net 6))
 (segment (start 86.4521 72.1165) (end 86.4521 67.9521) (width 0.5) (layer "B.Cu") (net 6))
 (segment (start 80 67) (end 70 67) (width 0.5) (layer "B.Cu") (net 6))
 (segment (start 86.4521 67.9521) (end 85.5 67) (width 0.5) (layer "B.Cu") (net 6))
 (segment (start 70 70.5) (end 69.5 71) (width 0.5) (layer "B.Cu") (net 6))
 (segment (start 80 67) (end 80 70.5) (width 0.5) (layer "B.Cu") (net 6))
 (segment (start 59.5 71) (end 57.4 71) (width 0.5) (layer "B.Cu") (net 6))
 (segment (start 60 70.5) (end 59.5 71) (width 0.5) (layer "B.Cu") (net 6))
 (segment (start 80 70.5) (end 79.5 71) (width 0.5) (layer "B.Cu") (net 6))
 (segment (start 70 67) (end 70 70.5) (width 0.5) (layer "B.Cu") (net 6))
 (segment (start 110.8928 86) (end 110.6788 85.786) (width 0.5) (layer "F.Cu") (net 9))
 (via (at 110.6788 85.786) (size 0.6) (drill 0.3) (layers "F.Cu" "B.Cu") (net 9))
 (segment (start 110.714 85.786) (end 110.928 86) (width 0.5) (layer "B.Cu") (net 9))
 (segment (start 110 86.4648) (end 110.6788 85.786) (width 0.5) (layer "B.Cu") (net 9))
 (segment (start 110 93.46) (end 110 86.4648) (width 0.5) (layer "B.Cu") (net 9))
 (segment (start 110.6788 85.786) (end 110.714 85.786) (width 0.5) (layer "B.Cu") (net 9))
 (segment (start 110.928 86) (end 124.92 86) (width 0.5) (layer "B.Cu") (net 9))
 (segment (start 110.4135 62.286) (end 116.286 62.286) (width 0.5) (layer "F.Cu") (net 12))
 (segment (start 116.286 62.286) (end 118.5 64.5) (width 0.5) (layer "F.Cu") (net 12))
 (segment (start 118.5 64.5) (end 118.5 87.5) (width 0.5) (layer "F.Cu") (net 12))
 (segment (start 124.92 62) (end 121 62) (width 0.5) (layer "F.Cu") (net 12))
 (segment (start 121 62) (end 118.5 64.5) (width 0.5) (layer "F.Cu") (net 12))
 (segment (start 118.5 87.5) (end 112.54 93.46) (width 0.5) (layer "F.Cu") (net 12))
 (segment (start 148.5 86) (end 146 88.5) (width 0.5) (layer "F.Cu") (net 13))
 (segment (start 146 88.5) (end 142 88.5) (width 0.5) (layer "F.Cu") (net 13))
 (segment (start 148.5 77.04) (end 148.5 86) (width 0.5) (layer "F.Cu") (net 13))
 (segment (start 144.5 73.04) (end 148.5 77.04) (width 0.5) (layer "F.Cu") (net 13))
 (segment (start 142 88.5) (end 140.48 90.02) (width 0.5) (layer "F.Cu") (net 13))
 (segment (start 140.48 90.02) (end 140.48 93.46) (width 0.5) (layer "F.Cu") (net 13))
 (via (at 110.6788 69.214) (size 0.6) (drill 0.3) (layers "F.Cu" "B.Cu") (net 2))
 (via (at 110.4135 57.714) (size 0.6) (drill 0.3) (layers "F.Cu" "B.Cu") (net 2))
 (via (at 110.6788 81.214) (size 0.6) (drill 0.3) (layers "F.Cu" "B.Cu") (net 2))
 (segment (start 153 70.5) (end 153 59) (width 0.5) (layer "B.Cu") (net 2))
 (segment (start 151.5 96) (end 153 94.5) (width 0.5) (layer "B.Cu") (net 2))
 (segment (start 110.6275 57.5) (end 110.4135 57.714) (width 0.5) (layer "B.Cu") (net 2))
 (segment (start 114 68) (end 112.786 69.214) (width 0.5) (layer "B.Cu") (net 2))
 (segment (start 112.786 69.214) (end 110.6788 69.214) (width 0.5) (layer "B.Cu") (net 2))
 (segment (start 153 59) (end 151.5 57.5) (width 0.5) (layer "B.Cu") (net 2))
 (segment (start 151.5 57.5) (end 114 57.5) (width 0.5) (layer "B.Cu") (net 2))
 (segment (start 114 57.5) (end 114 68) (width 0.5) (layer "B.Cu") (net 2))
 (segment (start 144.5 70.5) (end 153 70.5) (width 0.5) (layer "B.Cu") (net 2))
 (segment (start 148.1 96) (end 151.5 96) (width 0.5) (layer "B.Cu") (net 2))
 (segment (start 113.5 68.5) (end 113.5 80) (width 0.5) (layer "B.Cu") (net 2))
 (segment (start 113.5 80) (end 112.286 81.214) (width 0.5) (layer "B.Cu") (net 2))
 (segment (start 153 94.5) (end 153 70.5) (width 0.5) (layer "B.Cu") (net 2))
 (segment (start 114 57.5) (end 110.6275 57.5) (width 0.5) (layer "B.Cu") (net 2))
 (segment (start 114 68) (end 113.5 68.5) (width 0.5) (layer "B.Cu") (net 2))
 (segment (start 112.286 81.214) (end 110.6788 81.214) (width 0.5) (layer "B.Cu") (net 2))
 (segment (start 115.5 74.5) (end 115.5 87) (width 0.5) (layer "F.Cu") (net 1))
 (segment (start 108.5 89) (end 107.5 90) (width 0.5) (layer "F.Cu") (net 1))
 (segment (start 113.5 89) (end 108.5 89) (width 0.5) (layer "F.Cu") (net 1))
 (segment (start 114.786 73.786) (end 115.5 74.5) (width 0.5) (layer "F.Cu") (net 1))
 (segment (start 110.6788 73.786) (end 114.786 73.786) (width 0.5) (layer "F.Cu") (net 1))
 (segment (start 107.46 91.04) (end 107.46 93.46) (width 0.5) (layer "F.Cu") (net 1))
 (segment (start 115.5 87) (end 113.5 89) (width 0.5) (layer "F.Cu") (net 1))
 (segment (start 107.5 91) (end 107.46 91.04) (width 0.5) (layer "F.Cu") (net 1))
 (segment (start 107.5 90) (end 107.5 91) (width 0.5) (layer "F.Cu") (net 1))
 (via (at 115.5 74.5) (size 0.6) (drill 0.3) (layers "F.Cu" "B.Cu") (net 1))
 (segment (start 116 74) (end 115.5 74.5) (width 0.5) (layer "B.Cu") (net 1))
 (segment (start 136 87) (end 136 90) (width 0.5) (layer "F.Cu") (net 14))
 (segment (start 144.5 75.58) (end 140.92 75.58) (width 0.5) (layer "F.Cu") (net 14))
 (segment (start 130.32 91.18) (end 130.32 93.46) (width 0.5) (layer "F.Cu") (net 14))
 (segment (start 131.5 90) (end 130.32 91.18) (width 0.5) (layer "F.Cu") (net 14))
 (segment (start 139.5 83.5) (end 136 87) (width 0.5) (layer "F.Cu") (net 14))
 (segment (start 140.92 75.58) (end 139.5 77) (width 0.5) (layer "F.Cu") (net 14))
 (segment (start 139.5 77) (end 139.5 83.5) (width 0.5) (layer "F.Cu") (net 14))
 (segment (start 136 90) (end 131.5 90) (width 0.5) (layer "F.Cu") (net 14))
 (segment (start 147.5 87.5) (end 148.1 88.1) (width 0.5) (layer "B.Cu") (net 11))
 (segment (start 130 86) (end 131.5 87.5) (width 0.5) (layer "B.Cu") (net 11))
 (segment (start 148.1 88.1) (end 148.1 93.46) (width 0.5) (layer "B.Cu") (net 11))
 (segment (start 131.5 87.5) (end 147.5 87.5) (width 0.5) (layer "B.Cu") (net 11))
 (segment (start 101.8835 72.1165) (end 102.5 71.5) (width 0.5) (layer "F.Cu") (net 3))
 (segment (start 91.5321 72.1165) (end 101.8835 72.1165) (width 0.5) (layer "F.Cu") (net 3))
 (segment (start 91.5321 80.1165) (end 94.9156 83.5) (width 0.5) (layer "F.Cu") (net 10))
 (segment (start 94.9156 83.5) (end 102.5 83.5) (width 0.5) (layer "F.Cu") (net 10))
 (segment (start 91.6921 64.1165) (end 91.6921 62.3079) (width 0.5) (layer "F.Cu") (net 8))
 (segment (start 91.6921 62.3079) (end 94 60) (width 0.5) (layer "F.Cu") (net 8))
 (segment (start 94 60) (end 102.2347 60) (width 0.5) (layer "F.Cu") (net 8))
 (segment (start 144.5 78.12) (end 144.5 86) (width 0.5) (layer "F.Cu") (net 15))
 (segment (start 140 86) (end 137.94 88.06) (width 0.5) (layer "F.Cu") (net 15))
 (segment (start 144.5 86) (end 140 86) (width 0.5) (layer "F.Cu") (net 15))
 (segment (start 137.94 88.06) (end 137.94 93.46) (width 0.5) (layer "F.Cu") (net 15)))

